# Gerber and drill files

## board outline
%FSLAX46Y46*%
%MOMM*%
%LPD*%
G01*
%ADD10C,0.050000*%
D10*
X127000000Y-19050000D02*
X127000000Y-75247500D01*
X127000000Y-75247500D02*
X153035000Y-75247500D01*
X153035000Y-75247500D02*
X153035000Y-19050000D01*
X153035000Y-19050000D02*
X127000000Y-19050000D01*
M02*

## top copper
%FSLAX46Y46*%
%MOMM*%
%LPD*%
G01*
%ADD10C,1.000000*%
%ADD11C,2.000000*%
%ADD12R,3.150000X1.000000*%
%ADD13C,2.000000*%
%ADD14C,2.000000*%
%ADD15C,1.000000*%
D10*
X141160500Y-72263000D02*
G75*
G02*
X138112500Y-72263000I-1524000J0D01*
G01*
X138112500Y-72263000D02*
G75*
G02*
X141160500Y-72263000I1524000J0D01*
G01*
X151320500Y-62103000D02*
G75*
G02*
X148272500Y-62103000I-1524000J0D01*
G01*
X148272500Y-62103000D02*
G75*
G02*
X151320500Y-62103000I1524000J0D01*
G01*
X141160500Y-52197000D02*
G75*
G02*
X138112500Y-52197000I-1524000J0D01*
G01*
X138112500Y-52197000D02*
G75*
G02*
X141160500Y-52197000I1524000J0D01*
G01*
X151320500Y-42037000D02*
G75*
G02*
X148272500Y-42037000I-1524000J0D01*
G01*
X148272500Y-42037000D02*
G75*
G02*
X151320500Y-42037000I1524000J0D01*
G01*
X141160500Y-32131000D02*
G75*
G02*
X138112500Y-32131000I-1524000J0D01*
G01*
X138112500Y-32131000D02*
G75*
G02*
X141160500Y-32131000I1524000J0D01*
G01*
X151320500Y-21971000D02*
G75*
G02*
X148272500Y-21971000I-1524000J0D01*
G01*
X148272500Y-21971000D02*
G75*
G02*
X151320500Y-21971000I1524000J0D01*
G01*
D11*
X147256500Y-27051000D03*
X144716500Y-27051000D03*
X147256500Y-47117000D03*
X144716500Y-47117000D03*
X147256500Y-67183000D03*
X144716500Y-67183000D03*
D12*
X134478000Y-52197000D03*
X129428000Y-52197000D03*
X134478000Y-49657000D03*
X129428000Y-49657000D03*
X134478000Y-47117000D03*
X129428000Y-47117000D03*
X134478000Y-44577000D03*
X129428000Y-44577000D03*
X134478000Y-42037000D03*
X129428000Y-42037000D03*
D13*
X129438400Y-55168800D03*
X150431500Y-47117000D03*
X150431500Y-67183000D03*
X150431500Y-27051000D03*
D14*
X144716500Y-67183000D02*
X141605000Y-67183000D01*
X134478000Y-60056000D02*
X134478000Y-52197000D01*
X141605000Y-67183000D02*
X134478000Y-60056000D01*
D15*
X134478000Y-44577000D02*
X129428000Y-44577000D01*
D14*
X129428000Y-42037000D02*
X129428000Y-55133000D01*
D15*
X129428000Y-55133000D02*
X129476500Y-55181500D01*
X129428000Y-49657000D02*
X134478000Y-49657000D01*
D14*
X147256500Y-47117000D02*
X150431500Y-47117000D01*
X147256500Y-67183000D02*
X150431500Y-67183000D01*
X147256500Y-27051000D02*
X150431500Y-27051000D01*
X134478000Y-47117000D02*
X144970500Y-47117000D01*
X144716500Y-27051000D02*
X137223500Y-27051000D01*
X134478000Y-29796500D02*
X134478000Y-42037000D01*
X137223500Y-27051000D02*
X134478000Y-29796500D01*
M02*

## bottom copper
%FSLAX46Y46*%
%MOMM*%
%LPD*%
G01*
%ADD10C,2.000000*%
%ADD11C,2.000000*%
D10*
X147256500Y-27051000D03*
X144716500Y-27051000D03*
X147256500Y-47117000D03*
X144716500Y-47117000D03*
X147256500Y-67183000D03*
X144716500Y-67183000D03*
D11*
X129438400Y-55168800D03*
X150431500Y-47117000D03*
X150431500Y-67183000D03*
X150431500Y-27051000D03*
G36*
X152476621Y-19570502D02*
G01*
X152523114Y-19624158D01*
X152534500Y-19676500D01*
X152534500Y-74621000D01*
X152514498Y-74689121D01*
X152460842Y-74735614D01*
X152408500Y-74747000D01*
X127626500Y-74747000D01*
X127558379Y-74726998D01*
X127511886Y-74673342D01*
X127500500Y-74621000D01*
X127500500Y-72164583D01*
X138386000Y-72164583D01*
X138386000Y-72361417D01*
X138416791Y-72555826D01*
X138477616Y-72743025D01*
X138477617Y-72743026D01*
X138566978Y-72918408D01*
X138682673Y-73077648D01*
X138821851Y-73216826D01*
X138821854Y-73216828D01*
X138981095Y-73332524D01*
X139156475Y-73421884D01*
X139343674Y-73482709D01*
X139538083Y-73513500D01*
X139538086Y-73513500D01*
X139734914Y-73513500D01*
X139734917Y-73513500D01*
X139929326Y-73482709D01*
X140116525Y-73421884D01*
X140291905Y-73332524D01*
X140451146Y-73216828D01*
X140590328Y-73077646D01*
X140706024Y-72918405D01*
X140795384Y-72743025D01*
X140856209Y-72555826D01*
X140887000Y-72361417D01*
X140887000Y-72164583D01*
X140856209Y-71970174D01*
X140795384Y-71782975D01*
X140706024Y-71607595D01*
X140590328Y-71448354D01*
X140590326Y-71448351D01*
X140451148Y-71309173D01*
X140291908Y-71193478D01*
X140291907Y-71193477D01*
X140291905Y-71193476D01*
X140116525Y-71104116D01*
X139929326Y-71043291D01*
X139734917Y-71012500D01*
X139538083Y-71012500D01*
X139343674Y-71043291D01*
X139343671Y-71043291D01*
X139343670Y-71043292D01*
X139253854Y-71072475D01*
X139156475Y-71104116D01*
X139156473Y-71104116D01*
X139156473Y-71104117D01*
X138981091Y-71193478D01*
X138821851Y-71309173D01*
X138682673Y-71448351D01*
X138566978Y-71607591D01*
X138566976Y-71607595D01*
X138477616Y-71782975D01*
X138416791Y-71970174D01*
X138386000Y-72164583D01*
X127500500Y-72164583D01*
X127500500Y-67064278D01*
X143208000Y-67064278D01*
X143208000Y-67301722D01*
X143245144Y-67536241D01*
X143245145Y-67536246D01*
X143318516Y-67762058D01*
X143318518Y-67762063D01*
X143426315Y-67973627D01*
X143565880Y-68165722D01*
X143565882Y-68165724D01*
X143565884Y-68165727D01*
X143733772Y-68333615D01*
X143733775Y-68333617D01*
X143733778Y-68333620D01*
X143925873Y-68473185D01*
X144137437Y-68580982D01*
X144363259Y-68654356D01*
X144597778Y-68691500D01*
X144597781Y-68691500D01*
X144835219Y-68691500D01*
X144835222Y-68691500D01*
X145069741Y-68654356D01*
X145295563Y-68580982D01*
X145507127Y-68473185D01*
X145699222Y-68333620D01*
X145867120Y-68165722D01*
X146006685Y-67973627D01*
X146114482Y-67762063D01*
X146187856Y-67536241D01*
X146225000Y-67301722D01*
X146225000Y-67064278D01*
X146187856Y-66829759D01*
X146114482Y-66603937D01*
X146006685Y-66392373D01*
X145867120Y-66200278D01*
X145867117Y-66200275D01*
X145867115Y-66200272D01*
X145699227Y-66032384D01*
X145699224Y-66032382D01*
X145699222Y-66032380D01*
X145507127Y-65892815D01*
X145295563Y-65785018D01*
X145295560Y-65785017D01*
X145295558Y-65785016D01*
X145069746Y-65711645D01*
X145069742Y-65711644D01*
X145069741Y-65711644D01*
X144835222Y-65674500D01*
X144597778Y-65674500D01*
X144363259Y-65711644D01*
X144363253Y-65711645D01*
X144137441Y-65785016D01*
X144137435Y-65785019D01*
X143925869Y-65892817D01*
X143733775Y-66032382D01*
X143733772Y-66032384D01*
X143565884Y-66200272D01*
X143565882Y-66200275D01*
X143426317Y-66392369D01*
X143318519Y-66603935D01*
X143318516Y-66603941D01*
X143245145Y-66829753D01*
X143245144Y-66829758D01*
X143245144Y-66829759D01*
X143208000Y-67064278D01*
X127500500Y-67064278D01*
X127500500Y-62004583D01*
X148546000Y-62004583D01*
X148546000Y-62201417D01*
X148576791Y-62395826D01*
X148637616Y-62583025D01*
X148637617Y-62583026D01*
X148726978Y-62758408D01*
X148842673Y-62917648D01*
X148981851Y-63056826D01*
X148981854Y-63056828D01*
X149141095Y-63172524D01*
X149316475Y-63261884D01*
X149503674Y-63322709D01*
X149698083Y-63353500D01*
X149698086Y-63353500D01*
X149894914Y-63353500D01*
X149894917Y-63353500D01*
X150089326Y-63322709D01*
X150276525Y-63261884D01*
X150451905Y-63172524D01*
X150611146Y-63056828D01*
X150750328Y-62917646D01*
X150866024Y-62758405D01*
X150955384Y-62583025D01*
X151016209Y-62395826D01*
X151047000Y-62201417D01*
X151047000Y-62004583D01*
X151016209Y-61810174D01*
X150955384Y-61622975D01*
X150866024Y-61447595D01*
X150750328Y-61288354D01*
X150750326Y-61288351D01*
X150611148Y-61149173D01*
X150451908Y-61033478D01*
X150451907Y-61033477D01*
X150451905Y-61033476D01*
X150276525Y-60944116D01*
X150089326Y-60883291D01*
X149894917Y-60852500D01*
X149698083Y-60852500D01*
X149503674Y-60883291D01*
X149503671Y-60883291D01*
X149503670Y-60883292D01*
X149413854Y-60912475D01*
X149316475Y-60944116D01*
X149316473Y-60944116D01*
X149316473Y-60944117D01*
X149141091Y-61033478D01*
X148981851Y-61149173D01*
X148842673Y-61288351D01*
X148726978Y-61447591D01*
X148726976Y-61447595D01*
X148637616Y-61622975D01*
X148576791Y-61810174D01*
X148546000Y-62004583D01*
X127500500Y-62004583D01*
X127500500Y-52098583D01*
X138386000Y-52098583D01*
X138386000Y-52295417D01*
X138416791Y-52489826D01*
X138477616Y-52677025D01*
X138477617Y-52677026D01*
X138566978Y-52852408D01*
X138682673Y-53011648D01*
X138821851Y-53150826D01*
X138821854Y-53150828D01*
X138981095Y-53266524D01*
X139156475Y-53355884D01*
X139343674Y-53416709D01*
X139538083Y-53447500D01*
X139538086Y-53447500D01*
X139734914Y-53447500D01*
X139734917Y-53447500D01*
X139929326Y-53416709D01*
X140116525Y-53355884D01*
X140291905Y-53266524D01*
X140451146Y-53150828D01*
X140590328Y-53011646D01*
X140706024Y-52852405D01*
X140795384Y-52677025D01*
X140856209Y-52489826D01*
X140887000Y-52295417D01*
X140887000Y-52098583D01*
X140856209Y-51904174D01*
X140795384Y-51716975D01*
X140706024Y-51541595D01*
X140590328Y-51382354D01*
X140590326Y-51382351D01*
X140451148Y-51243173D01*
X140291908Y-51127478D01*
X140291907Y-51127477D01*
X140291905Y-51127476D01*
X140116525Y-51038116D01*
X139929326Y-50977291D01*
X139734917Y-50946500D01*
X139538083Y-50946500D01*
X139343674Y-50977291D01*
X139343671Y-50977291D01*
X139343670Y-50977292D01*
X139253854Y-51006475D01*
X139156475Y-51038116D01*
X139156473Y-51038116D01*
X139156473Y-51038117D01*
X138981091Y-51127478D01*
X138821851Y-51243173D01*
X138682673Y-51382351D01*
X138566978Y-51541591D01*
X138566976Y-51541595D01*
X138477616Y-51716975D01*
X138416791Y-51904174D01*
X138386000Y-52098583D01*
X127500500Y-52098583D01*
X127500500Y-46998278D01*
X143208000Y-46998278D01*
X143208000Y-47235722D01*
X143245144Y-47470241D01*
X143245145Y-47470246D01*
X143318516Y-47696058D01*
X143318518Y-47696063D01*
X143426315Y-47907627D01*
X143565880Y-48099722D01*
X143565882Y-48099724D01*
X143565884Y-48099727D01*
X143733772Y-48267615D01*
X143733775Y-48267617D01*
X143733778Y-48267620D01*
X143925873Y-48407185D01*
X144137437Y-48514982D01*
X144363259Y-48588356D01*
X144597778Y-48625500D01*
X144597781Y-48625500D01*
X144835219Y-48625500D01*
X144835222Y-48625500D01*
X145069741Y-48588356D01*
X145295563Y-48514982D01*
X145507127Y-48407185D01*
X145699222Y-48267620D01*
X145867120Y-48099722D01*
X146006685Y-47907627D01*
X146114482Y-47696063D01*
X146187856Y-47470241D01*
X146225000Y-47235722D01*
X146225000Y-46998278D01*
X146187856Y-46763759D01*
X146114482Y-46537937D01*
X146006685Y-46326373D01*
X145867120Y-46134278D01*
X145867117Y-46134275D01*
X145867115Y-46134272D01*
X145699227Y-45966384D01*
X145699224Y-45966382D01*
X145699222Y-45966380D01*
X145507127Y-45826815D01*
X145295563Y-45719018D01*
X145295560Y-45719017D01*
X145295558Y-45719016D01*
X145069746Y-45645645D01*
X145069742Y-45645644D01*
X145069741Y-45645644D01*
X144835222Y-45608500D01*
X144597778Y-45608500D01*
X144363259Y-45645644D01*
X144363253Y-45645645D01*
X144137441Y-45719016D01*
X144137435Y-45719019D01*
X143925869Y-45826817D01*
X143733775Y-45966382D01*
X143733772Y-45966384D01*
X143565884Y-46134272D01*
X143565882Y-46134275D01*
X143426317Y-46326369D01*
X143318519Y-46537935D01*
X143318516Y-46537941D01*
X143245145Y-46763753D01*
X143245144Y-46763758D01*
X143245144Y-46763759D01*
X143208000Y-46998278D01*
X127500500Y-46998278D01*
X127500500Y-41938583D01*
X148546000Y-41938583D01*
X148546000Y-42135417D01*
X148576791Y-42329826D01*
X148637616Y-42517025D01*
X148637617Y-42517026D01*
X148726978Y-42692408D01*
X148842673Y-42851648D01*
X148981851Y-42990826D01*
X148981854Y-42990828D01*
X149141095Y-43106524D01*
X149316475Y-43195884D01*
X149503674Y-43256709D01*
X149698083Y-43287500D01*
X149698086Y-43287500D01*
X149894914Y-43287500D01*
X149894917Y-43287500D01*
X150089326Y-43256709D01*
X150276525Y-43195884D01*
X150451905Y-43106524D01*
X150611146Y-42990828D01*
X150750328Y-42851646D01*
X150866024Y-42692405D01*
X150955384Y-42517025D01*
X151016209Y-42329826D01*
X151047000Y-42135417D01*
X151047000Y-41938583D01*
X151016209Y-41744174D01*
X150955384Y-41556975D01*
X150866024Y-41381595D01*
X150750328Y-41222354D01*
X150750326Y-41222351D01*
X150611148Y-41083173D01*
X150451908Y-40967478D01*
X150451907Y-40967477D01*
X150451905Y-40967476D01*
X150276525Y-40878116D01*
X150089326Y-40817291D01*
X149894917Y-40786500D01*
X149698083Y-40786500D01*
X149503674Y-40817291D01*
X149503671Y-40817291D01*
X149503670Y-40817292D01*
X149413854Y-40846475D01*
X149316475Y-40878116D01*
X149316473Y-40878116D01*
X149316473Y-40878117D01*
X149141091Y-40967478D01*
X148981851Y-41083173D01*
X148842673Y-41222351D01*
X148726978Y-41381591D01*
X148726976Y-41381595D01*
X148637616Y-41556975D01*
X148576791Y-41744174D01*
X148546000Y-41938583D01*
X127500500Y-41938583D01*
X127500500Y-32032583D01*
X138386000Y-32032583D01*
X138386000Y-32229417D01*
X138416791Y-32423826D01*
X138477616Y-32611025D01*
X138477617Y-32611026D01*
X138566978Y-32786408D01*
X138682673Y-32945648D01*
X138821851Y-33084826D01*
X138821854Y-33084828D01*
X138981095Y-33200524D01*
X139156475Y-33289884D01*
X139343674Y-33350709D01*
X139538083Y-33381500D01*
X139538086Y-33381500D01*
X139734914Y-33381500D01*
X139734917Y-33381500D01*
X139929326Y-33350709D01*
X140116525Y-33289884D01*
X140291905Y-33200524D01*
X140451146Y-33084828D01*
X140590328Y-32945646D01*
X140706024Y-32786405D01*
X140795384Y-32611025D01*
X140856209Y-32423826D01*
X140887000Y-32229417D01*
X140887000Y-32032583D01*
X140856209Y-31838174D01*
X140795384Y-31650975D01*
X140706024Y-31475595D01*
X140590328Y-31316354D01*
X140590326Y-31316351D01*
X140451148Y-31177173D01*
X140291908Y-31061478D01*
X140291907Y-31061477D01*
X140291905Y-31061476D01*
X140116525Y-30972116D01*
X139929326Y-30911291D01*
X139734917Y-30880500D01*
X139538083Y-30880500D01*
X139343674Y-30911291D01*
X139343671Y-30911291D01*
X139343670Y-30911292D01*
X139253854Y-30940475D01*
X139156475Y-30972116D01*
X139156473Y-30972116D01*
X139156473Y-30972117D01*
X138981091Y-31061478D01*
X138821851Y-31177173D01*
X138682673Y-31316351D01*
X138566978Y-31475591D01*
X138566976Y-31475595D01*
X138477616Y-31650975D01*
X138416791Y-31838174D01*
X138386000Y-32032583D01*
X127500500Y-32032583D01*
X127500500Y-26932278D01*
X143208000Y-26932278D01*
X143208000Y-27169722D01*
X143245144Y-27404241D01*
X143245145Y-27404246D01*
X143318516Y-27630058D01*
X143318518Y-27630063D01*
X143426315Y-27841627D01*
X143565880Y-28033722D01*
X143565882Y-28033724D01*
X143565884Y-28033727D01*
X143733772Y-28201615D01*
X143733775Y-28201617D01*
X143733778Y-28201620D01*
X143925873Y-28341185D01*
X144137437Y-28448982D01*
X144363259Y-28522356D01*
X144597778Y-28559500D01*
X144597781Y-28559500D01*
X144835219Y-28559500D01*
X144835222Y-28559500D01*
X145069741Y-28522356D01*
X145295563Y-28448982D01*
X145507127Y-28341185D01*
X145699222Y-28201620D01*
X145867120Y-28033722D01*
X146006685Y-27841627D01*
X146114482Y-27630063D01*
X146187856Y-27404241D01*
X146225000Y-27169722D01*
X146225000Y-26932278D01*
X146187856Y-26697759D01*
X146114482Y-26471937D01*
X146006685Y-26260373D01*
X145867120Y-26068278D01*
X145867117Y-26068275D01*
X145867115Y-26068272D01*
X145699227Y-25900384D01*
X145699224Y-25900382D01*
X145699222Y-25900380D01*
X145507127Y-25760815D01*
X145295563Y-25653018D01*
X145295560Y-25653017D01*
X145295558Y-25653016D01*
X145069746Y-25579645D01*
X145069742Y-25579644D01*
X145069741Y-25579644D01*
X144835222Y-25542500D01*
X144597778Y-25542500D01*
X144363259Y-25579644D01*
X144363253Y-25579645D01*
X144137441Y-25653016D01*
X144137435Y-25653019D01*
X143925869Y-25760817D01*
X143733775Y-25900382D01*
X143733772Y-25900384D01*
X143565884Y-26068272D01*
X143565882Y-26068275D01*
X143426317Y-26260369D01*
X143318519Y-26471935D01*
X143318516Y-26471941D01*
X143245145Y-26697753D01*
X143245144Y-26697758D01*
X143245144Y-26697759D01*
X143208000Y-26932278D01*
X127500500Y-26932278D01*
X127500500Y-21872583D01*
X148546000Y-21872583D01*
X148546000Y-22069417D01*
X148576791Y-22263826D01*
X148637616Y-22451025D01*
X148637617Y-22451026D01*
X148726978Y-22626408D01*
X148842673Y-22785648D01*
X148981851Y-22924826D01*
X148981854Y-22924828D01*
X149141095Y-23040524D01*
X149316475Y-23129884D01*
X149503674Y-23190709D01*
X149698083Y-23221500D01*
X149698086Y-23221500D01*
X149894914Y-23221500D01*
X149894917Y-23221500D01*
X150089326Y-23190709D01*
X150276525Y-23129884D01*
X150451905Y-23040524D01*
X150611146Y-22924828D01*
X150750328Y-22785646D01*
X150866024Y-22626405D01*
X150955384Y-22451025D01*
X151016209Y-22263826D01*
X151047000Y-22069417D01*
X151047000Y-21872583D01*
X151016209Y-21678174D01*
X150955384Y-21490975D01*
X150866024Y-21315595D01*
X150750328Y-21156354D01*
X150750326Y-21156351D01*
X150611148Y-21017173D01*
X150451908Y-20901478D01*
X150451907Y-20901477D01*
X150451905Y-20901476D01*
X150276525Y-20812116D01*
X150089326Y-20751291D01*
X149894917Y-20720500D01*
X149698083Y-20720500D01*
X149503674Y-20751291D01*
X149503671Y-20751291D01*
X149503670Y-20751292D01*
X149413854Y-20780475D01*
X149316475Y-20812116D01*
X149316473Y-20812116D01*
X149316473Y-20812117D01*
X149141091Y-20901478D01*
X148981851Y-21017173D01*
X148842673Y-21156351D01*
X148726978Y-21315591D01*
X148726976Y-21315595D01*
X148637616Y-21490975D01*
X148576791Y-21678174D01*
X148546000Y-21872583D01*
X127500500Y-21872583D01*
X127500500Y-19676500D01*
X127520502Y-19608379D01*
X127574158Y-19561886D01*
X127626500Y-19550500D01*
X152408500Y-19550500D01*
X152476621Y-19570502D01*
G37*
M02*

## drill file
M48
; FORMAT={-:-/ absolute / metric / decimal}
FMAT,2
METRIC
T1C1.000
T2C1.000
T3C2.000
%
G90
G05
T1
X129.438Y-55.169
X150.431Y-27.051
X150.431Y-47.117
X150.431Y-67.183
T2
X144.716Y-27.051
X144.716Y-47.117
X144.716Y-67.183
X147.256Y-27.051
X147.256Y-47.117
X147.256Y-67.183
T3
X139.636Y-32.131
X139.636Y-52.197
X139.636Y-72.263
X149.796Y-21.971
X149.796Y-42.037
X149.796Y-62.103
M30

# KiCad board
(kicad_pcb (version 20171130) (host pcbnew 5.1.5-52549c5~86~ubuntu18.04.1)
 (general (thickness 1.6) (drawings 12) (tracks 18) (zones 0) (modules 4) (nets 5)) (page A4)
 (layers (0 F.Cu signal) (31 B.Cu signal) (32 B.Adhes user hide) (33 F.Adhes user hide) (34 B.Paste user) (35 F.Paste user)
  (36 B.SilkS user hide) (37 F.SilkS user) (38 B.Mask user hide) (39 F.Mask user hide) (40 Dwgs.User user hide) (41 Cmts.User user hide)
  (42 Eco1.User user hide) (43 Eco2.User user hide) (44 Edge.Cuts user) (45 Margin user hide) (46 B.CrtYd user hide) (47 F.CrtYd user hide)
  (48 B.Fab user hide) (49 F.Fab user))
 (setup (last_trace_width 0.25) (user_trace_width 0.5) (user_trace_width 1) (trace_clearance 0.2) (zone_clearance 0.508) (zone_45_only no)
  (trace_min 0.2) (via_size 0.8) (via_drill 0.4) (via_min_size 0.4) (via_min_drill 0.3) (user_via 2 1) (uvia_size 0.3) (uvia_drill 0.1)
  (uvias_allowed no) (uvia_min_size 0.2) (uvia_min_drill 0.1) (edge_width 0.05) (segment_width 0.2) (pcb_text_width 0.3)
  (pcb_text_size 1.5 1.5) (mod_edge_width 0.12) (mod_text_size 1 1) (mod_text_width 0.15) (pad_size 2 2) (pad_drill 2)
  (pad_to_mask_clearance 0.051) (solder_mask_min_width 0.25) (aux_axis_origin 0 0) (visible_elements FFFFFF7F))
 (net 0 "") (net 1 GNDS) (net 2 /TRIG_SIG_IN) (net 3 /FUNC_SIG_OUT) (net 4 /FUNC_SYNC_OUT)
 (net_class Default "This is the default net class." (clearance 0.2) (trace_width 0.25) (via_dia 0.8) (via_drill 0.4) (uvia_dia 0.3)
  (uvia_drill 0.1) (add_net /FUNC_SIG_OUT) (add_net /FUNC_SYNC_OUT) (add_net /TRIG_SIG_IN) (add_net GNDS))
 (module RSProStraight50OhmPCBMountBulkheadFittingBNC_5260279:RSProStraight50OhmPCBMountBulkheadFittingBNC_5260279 (layer F.Cu)
  (at 144.7165 27.051 180)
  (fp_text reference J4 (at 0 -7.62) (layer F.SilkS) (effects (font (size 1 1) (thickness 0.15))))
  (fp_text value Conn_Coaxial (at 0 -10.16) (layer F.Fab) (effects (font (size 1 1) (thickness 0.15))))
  (pad 2 thru_hole circle (at -2.54 0 180) (size 2 2) (drill 1) (layers *.Cu *.Mask) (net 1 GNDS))
  (pad 1 thru_hole circle (at 0 0 180) (size 2 2) (drill 1) (layers *.Cu *.Mask) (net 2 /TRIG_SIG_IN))
  (pad "" np_thru_hole circle (at -5.08 5.08 180) (size 2 2) (drill 2) (layers *.Cu *.Mask))
  (pad "" np_thru_hole circle (at 5.08 -5.08 180) (size 2 2) (drill 2) (layers *.Cu *.Mask)))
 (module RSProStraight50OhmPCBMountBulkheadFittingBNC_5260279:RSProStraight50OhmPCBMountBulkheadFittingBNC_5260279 (layer F.Cu)
  (at 144.7165 47.117 180)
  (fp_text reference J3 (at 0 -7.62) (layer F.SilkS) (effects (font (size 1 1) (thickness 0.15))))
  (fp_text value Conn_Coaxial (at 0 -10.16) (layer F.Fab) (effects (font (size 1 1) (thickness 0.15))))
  (pad 2 thru_hole circle (at -2.54 0 180) (size 2 2) (drill 1) (layers *.Cu *.Mask) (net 1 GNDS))
  (pad 1 thru_hole circle (at 0 0 180) (size 2 2) (drill 1) (layers *.Cu *.Mask) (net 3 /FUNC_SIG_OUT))
  (pad "" np_thru_hole circle (at -5.08 5.08 180) (size 2 2) (drill 2) (layers *.Cu *.Mask))
  (pad "" np_thru_hole circle (at 5.08 -5.08 180) (size 2 2) (drill 2) (layers *.Cu *.Mask)))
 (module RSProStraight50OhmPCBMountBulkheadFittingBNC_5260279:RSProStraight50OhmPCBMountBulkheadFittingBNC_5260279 (layer F.Cu)
  (at 144.7165 67.183 180)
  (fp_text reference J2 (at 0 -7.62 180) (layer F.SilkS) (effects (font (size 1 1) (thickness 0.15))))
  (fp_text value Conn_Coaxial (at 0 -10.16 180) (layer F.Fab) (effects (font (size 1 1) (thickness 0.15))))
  (pad 2 thru_hole circle (at -2.54 0 180) (size 2 2) (drill 1) (layers *.Cu *.Mask) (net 1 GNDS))
  (pad 1 thru_hole circle (at 0 0 180) (size 2 2) (drill 1) (layers *.Cu *.Mask) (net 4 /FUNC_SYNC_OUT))
  (pad "" np_thru_hole circle (at -5.08 5.08 180) (size 2 2) (drill 2) (layers *.Cu *.Mask))
  (pad "" np_thru_hole circle (at 5.08 -5.08 180) (size 2 2) (drill 2) (layers *.Cu *.Mask)))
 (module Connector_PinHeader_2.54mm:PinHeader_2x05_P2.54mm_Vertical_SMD (layer F.Cu) (at 131.953 47.117 180)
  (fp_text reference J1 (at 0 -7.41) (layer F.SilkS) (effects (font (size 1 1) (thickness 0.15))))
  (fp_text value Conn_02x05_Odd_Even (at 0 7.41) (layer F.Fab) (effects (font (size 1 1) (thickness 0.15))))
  (pad 1 smd rect (at -2.525 -5.08 180) (size 3.15 1) (layers F.Cu F.Paste F.Mask) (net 4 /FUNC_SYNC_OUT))
  (pad 2 smd rect (at 2.525 -5.08 180) (size 3.15 1) (layers F.Cu F.Paste F.Mask) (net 1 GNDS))
  (pad 3 smd rect (at -2.525 -2.54 180) (size 3.15 1) (layers F.Cu F.Paste F.Mask) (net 1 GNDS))
  (pad 4 smd rect (at 2.525 -2.54 180) (size 3.15 1) (layers F.Cu F.Paste F.Mask) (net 1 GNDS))
  (pad 5 smd rect (at -2.525 0 180) (size 3.15 1) (layers F.Cu F.Paste F.Mask) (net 3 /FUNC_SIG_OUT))
  (pad 6 smd rect (at 2.525 0 180) (size 3.15 1) (layers F.Cu F.Paste F.Mask) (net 1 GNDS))
  (pad 7 smd rect (at -2.525 2.54 180) (size 3.15 1) (layers F.Cu F.Paste F.Mask) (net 1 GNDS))
  (pad 8 smd rect (at 2.525 2.54 180) (size 3.15 1) (layers F.Cu F.Paste F.Mask) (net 1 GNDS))
  (pad 9 smd rect (at -2.525 5.08 180) (size 3.15 1) (layers F.Cu F.Paste F.Mask) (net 2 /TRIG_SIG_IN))
  (pad 10 smd rect (at 2.525 5.08 180) (size 3.15 1) (layers F.Cu F.Paste F.Mask) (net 1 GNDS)))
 (gr_circle (center 139.6365 72.263) (end 141.1605 72.263) (layer F.Cu) (width 1))
 (gr_circle (center 149.7965 62.103) (end 151.3205 62.103) (layer F.Cu) (width 1))
 (gr_circle (center 139.6365 52.197) (end 141.1605 52.197) (layer F.Cu) (width 1))
 (gr_circle (center 149.7965 42.037) (end 151.3205 42.037) (layer F.Cu) (width 1))
 (gr_circle (center 139.6365 32.131) (end 141.1605 32.131) (layer F.Cu) (width 1))
 (gr_circle (center 149.7965 21.971) (end 151.3205 21.971) (layer F.Cu) (width 1))
 (gr_line (start 127 19.05) (end 127 75.2475) (layer Edge.Cuts) (width 0.05))
 (gr_line (start 127 75.2475) (end 153.035 75.2475) (layer Edge.Cuts) (width 0.05))
 (gr_line (start 153.035 75.2475) (end 153.035 19.05) (layer Edge.Cuts) (width 0.05))
 (gr_line (start 153.035 19.05) (end 127 19.05) (layer Edge.Cuts) (width 0.05))
 (segment (start 144.7165 67.183) (end 141.605 67.183) (width 2) (layer F.Cu) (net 4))
 (segment (start 134.478 60.056) (end 134.478 52.197) (width 2) (layer F.Cu) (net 4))
 (segment (start 141.605 67.183) (end 134.478 60.056) (width 2) (layer F.Cu) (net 4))
 (segment (start 134.478 44.577) (end 129.428 44.577) (width 1) (layer F.Cu) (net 1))
 (segment (start 129.428 42.037) (end 129.428 55.133) (width 2) (layer F.Cu) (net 1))
 (via (at 129.4384 55.1688) (size 2) (drill 1) (layers F.Cu B.Cu) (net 1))
 (segment (start 129.428 55.133) (end 129.4765 55.1815) (width 1) (layer F.Cu) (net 1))
 (segment (start 129.428 49.657) (end 134.478 49.657) (width 1) (layer F.Cu) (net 1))
 (segment (start 147.2565 47.117) (end 150.4315 47.117) (width 2) (layer F.Cu) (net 1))
 (via (at 150.4315 47.117) (size 2) (drill 1) (layers F.Cu B.Cu) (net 1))
 (segment (start 147.2565 67.183) (end 150.4315 67.183) (width 2) (layer F.Cu) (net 1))
 (via (at 150.4315 67.183) (size 2) (drill 1) (layers F.Cu B.Cu) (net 1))
 (segment (start 147.2565 27.051) (end 150.4315 27.051) (width 2) (layer F.Cu) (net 1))
 (via (at 150.4315 27.051) (size 2) (drill 1) (layers F.Cu B.Cu) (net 1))
 (segment (start 134.478 47.117) (end 144.9705 47.117) (width 2) (layer F.Cu) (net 3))
 (segment (start 144.7165 27.051) (end 137.2235 27.051) (width 2) (layer F.Cu) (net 2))
 (segment (start 134.478 29.7965) (end 134.478 42.037) (width 2) (layer F.Cu) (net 2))
 (segment (start 137.2235 27.051) (end 134.478 29.7965) (width 2) (layer F.Cu) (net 2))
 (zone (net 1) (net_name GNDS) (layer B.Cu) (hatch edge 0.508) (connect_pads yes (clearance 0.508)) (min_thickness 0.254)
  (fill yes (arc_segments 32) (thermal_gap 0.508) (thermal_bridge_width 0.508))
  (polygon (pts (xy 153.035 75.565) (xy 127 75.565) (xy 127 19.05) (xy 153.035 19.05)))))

